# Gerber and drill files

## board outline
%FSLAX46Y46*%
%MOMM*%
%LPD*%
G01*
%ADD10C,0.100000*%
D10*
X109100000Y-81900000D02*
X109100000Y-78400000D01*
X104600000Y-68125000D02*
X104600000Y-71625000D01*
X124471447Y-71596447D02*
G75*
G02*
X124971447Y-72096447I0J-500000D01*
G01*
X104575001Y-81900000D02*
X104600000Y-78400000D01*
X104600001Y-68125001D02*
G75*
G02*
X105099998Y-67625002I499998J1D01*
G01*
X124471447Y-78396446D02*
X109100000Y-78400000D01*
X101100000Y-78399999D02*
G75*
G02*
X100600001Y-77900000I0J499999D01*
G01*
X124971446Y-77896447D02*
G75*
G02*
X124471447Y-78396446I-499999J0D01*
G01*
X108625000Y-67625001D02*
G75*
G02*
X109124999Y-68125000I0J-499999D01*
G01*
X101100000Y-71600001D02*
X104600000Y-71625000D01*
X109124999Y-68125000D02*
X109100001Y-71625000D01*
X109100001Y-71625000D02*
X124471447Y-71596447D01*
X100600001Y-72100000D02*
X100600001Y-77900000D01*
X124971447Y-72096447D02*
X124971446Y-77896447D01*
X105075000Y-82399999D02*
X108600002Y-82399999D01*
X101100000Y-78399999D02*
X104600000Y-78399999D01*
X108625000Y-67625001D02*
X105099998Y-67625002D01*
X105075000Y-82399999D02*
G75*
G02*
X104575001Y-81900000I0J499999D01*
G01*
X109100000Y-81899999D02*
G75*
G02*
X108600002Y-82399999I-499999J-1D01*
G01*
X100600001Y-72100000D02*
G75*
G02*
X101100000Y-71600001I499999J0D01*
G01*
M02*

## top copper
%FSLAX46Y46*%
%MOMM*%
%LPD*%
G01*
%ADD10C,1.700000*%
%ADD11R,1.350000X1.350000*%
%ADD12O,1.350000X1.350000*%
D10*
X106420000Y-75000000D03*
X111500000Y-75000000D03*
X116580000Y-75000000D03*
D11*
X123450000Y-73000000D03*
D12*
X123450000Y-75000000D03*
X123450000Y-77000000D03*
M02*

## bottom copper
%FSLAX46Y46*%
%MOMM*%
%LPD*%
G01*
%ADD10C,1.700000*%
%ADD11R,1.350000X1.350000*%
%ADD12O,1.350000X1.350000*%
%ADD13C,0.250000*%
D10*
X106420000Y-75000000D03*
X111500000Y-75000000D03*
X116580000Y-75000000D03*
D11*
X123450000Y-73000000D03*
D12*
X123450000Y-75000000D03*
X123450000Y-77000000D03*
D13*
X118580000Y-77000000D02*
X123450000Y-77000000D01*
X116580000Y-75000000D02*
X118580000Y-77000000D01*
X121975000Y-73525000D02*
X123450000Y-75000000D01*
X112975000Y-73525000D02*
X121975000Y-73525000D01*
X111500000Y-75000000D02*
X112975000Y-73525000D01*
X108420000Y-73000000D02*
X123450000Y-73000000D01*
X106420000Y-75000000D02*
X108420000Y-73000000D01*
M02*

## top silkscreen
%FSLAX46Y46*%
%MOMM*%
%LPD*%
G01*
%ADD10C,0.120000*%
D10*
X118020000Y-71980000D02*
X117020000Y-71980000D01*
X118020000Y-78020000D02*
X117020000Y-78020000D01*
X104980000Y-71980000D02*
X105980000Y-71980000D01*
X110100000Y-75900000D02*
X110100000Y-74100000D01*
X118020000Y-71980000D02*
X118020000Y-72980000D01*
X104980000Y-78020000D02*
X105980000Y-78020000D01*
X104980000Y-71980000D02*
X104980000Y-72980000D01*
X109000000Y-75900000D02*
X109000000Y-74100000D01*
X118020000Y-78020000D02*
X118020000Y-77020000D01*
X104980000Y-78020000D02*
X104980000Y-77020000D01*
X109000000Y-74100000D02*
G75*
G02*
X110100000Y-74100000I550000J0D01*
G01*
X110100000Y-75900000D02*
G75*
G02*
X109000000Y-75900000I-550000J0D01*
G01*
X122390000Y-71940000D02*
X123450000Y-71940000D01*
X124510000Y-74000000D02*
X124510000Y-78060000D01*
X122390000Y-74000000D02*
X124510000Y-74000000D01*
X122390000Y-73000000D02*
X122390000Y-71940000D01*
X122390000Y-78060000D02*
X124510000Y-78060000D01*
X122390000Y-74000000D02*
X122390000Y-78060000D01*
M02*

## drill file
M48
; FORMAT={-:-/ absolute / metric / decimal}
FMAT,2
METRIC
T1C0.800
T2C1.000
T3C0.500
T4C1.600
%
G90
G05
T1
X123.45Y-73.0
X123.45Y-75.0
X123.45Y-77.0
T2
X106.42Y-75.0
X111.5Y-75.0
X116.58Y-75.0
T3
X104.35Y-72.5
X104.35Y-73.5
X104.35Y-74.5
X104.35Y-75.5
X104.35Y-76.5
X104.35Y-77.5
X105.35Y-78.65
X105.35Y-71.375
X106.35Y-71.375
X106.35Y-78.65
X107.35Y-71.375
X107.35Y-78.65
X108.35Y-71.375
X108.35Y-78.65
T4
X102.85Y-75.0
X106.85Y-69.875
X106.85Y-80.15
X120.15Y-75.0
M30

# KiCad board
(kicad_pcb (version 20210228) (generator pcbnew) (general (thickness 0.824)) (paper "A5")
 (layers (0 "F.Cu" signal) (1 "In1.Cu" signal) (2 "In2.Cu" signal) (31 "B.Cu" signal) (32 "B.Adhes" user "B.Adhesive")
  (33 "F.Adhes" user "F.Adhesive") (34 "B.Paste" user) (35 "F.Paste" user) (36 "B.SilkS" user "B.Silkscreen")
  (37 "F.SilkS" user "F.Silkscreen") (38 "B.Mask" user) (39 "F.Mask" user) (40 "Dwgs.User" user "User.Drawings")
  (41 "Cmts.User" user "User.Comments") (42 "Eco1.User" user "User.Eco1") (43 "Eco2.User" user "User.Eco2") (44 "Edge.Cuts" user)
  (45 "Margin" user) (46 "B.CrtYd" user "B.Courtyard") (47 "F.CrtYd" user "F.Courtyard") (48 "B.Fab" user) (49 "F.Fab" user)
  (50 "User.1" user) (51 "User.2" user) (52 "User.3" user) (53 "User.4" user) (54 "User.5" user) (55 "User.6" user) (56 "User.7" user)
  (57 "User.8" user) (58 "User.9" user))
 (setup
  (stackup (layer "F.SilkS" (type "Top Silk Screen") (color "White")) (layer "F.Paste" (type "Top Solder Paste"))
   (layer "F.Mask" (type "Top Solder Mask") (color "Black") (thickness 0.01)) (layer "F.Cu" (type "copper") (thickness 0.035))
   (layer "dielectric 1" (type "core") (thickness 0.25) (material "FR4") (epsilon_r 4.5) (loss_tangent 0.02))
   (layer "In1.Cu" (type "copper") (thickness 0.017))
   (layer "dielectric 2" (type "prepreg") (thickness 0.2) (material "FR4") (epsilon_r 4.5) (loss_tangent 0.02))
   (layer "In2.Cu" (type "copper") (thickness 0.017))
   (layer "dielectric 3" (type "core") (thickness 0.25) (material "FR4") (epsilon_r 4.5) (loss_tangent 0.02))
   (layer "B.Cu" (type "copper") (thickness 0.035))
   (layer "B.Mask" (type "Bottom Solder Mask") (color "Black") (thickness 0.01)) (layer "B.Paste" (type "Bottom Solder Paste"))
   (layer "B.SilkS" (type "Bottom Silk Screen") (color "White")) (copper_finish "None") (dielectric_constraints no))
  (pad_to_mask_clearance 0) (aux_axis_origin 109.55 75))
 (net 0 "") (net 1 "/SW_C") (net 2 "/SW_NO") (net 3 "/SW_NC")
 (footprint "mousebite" (layer "F.Cu") (at 104.35 73.5)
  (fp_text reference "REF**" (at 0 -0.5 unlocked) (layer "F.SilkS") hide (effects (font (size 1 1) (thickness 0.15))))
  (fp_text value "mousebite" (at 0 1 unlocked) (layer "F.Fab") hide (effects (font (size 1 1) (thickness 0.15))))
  (pad "" np_thru_hole circle (at 0 0) (size 0.5 0.5) (drill 0.5) (layers F&B.Cu *.Mask)))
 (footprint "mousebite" (layer "F.Cu") (at 105.350001 71.375 -90)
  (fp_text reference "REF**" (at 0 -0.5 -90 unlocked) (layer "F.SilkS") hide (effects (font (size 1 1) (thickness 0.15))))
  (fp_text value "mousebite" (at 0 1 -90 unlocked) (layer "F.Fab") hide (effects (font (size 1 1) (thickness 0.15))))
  (pad "" np_thru_hole circle (at 0 0 270) (size 0.5 0.5) (drill 0.5) (layers F&B.Cu *.Mask)))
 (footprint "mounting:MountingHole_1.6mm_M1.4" (layer "F.Cu") (at 106.85 69.875001 -90)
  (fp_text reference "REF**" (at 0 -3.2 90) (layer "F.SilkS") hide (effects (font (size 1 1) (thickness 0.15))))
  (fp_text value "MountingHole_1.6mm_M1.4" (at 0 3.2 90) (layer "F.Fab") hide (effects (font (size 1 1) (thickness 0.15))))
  (pad "" np_thru_hole circle (at 0 0 270) (locked) (size 1.6 1.6) (drill 1.6) (layers F&B.Cu *.Mask)))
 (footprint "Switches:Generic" (layer "F.Cu") (at 111.5 75)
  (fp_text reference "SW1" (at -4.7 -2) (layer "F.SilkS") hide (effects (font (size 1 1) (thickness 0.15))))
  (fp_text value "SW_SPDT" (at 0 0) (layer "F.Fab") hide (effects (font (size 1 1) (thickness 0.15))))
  (fp_line (start 6.52 -3.02) (end 5.52 -3.02) (layer "F.SilkS") (width 0.12))
  (fp_line (start 6.52 3.02) (end 5.52 3.02) (layer "F.SilkS") (width 0.12))
  (fp_line (start -6.52 -3.02) (end -5.52 -3.02) (layer "F.SilkS") (width 0.12))
  (fp_line (start -1.4 0.9) (end -1.4 -0.9) (layer "F.SilkS") (width 0.12))
  (fp_line (start 6.52 -3.02) (end 6.52 -2.02) (layer "F.SilkS") (width 0.12))
  (fp_line (start -6.52 3.02) (end -5.52 3.02) (layer "F.SilkS") (width 0.12))
  (fp_line (start -6.52 -3.02) (end -6.52 -2.02) (layer "F.SilkS") (width 0.12))
  (fp_line (start -2.5 0.9) (end -2.5 -0.9) (layer "F.SilkS") (width 0.12))
  (fp_line (start 6.52 3.02) (end 6.52 2.02) (layer "F.SilkS") (width 0.12))
  (fp_line (start -6.52 3.02) (end -6.52 2.02) (layer "F.SilkS") (width 0.12))
  (fp_arc (start -1.95 -0.9) (end -1.4 -0.9) (angle -180) (layer "F.SilkS") (width 0.12))
  (fp_arc (start -1.95 0.9) (end -2.5 0.9) (angle -180) (layer "F.SilkS") (width 0.12))
  (pad "1" thru_hole circle (at -5.08 0) (locked) (size 1.7 1.7) (drill 1) (layers *.Cu *.Mask) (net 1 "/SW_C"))
  (pad "2" thru_hole circle (at 0 0) (locked) (size 1.7 1.7) (drill 1) (layers *.Cu *.Mask) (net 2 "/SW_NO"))
  (pad "3" thru_hole circle (at 5.08 0) (locked) (size 1.7 1.7) (drill 1) (layers *.Cu *.Mask) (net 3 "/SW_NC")))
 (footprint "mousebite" (layer "F.Cu") (at 104.35 75.5)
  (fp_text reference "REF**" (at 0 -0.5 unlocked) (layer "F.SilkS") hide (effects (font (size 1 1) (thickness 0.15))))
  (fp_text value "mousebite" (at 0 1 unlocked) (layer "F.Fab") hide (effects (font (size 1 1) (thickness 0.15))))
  (pad "" np_thru_hole circle (at 0 0) (size 0.5 0.5) (drill 0.5) (layers F&B.Cu *.Mask)))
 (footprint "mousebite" (layer "F.Cu") (at 104.35 74.5)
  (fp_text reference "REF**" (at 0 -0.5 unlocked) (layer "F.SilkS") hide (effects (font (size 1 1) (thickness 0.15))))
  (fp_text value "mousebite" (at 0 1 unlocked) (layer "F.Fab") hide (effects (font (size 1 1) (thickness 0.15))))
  (pad "" np_thru_hole circle (at 0 0) (size 0.5 0.5) (drill 0.5) (layers F&B.Cu *.Mask)))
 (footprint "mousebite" (layer "F.Cu") (at 104.35 76.5)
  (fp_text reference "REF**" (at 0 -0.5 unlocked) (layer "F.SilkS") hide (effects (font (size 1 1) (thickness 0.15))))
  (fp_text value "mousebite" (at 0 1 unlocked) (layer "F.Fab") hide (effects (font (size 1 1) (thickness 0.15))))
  (pad "" np_thru_hole circle (at 0 0) (size 0.5 0.5) (drill 0.5) (layers F&B.Cu *.Mask)))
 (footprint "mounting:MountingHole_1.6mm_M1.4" (layer "F.Cu") (at 120.15 75)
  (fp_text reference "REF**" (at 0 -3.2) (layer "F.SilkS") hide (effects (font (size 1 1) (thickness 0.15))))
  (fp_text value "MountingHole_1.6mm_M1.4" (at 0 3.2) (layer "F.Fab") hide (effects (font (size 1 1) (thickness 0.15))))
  (pad "" np_thru_hole circle (at 0 0) (locked) (size 1.6 1.6) (drill 1.6) (layers F&B.Cu *.Mask)))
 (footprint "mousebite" (layer "F.Cu") (at 104.35 72.5)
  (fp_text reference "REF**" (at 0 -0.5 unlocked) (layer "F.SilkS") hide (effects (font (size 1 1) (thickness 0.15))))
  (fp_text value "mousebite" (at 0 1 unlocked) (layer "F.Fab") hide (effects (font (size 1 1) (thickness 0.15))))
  (pad "" np_thru_hole circle (at 0 0) (size 0.5 0.5) (drill 0.5) (layers F&B.Cu *.Mask)))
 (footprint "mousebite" (layer "F.Cu") (at 107.35 78.65 90)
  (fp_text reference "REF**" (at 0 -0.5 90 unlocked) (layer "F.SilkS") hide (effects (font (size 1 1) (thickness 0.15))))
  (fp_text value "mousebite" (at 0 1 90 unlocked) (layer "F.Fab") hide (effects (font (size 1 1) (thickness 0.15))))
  (pad "" np_thru_hole circle (at 0 0 90) (size 0.5 0.5) (drill 0.5) (layers F&B.Cu *.Mask)))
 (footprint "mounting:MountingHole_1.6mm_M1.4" (layer "F.Cu") (at 102.85 75)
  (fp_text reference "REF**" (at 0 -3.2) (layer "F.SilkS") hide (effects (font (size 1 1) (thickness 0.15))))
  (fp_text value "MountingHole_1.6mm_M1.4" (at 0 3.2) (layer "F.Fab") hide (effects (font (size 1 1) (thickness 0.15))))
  (pad "" np_thru_hole circle (at 0 0) (locked) (size 1.6 1.6) (drill 1.6) (layers F&B.Cu *.Mask)))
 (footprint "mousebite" (layer "F.Cu") (at 108.349999 78.65 90)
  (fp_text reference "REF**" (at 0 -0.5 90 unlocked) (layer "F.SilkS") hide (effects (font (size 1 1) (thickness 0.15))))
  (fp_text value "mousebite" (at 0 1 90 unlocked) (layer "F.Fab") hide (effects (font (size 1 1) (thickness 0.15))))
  (pad "" np_thru_hole circle (at 0 0 90) (size 0.5 0.5) (drill 0.5) (layers F&B.Cu *.Mask)))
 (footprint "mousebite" (layer "F.Cu") (at 107.35 71.375 -90)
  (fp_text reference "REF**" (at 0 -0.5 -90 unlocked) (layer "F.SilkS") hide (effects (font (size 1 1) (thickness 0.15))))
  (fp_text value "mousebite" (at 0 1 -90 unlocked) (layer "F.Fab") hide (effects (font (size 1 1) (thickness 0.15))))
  (pad "" np_thru_hole circle (at 0 0 270) (size 0.5 0.5) (drill 0.5) (layers F&B.Cu *.Mask)))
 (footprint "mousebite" (layer "F.Cu") (at 106.35 78.65 90)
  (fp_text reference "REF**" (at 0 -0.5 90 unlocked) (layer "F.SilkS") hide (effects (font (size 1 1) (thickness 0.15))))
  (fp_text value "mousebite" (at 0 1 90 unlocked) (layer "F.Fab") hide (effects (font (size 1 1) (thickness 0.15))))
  (pad "" np_thru_hole circle (at 0 0 90) (size 0.5 0.5) (drill 0.5) (layers F&B.Cu *.Mask)))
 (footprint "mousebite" (layer "F.Cu") (at 105.35 78.65 90)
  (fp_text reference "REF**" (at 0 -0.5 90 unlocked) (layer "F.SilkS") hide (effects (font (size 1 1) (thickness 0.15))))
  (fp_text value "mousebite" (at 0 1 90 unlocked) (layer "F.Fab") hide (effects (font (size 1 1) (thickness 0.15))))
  (pad "" np_thru_hole circle (at 0 0 90) (size 0.5 0.5) (drill 0.5) (layers F&B.Cu *.Mask)))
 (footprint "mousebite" (layer "F.Cu") (at 106.35 71.375 -90)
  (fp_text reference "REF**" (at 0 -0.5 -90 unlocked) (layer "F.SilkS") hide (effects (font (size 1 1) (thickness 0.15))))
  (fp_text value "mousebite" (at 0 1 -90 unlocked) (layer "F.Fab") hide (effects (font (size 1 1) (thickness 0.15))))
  (pad "" np_thru_hole circle (at 0 0 270) (size 0.5 0.5) (drill 0.5) (layers F&B.Cu *.Mask)))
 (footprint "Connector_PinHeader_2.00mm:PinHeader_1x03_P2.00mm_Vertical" (layer "F.Cu") (at 123.45 73)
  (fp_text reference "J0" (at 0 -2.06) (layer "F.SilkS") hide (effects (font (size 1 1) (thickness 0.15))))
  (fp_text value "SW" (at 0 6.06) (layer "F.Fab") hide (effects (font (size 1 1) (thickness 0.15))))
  (fp_line (start -1.06 -1.06) (end 0 -1.06) (layer "F.SilkS") (width 0.12))
  (fp_line (start 1.06 1) (end 1.06 5.06) (layer "F.SilkS") (width 0.12))
  (fp_line (start -1.06 1) (end 1.06 1) (layer "F.SilkS") (width 0.12))
  (fp_line (start -1.06 0) (end -1.06 -1.06) (layer "F.SilkS") (width 0.12))
  (fp_line (start -1.06 5.06) (end 1.06 5.06) (layer "F.SilkS") (width 0.12))
  (fp_line (start -1.06 1) (end -1.06 5.06) (layer "F.SilkS") (width 0.12))
  (pad "1" thru_hole rect (at 0 0) (locked) (size 1.35 1.35) (drill 0.8) (layers *.Cu *.Mask) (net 1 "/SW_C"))
  (pad "2" thru_hole oval (at 0 2) (locked) (size 1.35 1.35) (drill 0.8) (layers *.Cu *.Mask) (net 2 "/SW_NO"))
  (pad "3" thru_hole oval (at 0 4) (locked) (size 1.35 1.35) (drill 0.8) (layers *.Cu *.Mask) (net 3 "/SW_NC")))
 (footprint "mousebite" (layer "F.Cu") (at 108.349999 71.375 -90)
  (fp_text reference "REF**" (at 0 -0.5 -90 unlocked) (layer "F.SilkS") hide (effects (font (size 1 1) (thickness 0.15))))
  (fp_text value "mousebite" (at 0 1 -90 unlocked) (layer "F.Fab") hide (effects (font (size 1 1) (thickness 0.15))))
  (pad "" np_thru_hole circle (at 0 0 270) (size 0.5 0.5) (drill 0.5) (layers F&B.Cu *.Mask)))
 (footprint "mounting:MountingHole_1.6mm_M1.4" (layer "F.Cu") (at 106.85 80.149999 90)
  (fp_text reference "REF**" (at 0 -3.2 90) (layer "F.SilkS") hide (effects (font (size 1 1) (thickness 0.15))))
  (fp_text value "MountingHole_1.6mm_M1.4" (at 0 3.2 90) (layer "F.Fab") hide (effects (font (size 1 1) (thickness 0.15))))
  (pad "" np_thru_hole circle (at 0 0 90) (locked) (size 1.6 1.6) (drill 1.6) (layers F&B.Cu *.Mask)))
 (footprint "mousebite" (layer "F.Cu") (at 104.35 77.5)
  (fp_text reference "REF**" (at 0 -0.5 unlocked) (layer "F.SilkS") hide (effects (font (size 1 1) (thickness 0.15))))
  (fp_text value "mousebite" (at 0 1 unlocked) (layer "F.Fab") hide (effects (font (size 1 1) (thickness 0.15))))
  (pad "" np_thru_hole circle (at 0 0) (size 0.5 0.5) (drill 0.5) (layers F&B.Cu *.Mask)))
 (gr_line (start 109.1 81.9) (end 109.1 78.4) (layer "Edge.Cuts") (width 0.1))
 (gr_line (start 104.6 68.125) (end 104.6 71.625) (layer "Edge.Cuts") (width 0.1))
 (gr_arc (start 124.471447 72.096447) (end 124.971447 72.096447) (angle -90) (layer "Edge.Cuts") (width 0.1))
 (gr_line (start 104.575001 81.9) (end 104.6 78.4) (layer "Edge.Cuts") (width 0.1))
 (gr_arc (start 105.099999 68.125) (end 105.099998 67.625002) (angle -90) (layer "Edge.Cuts") (width 0.1))
 (gr_line (start 124.471447 78.396446) (end 109.1 78.4) (layer "Edge.Cuts") (width 0.1))
 (gr_arc (start 101.1 77.9) (end 100.600001 77.9) (angle -90) (layer "Edge.Cuts") (width 0.1))
 (gr_arc (start 124.471447 77.896447) (end 124.471447 78.396446) (angle -90) (layer "Edge.Cuts") (width 0.1))
 (gr_arc (start 108.625 68.125) (end 109.124999 68.125) (angle -90) (layer "Edge.Cuts") (width 0.1))
 (gr_line (start 101.1 71.600001) (end 104.6 71.625) (layer "Edge.Cuts") (width 0.1))
 (gr_line (start 109.124999 68.125) (end 109.100001 71.625) (layer "Edge.Cuts") (width 0.1))
 (gr_line (start 109.100001 71.625) (end 124.471447 71.596447) (layer "Edge.Cuts") (width 0.1))
 (gr_line (start 100.600001 72.1) (end 100.600001 77.9) (layer "Edge.Cuts") (width 0.1))
 (gr_line (start 124.971447 72.096447) (end 124.971446 77.896447) (layer "Edge.Cuts") (width 0.1))
 (gr_line (start 105.075 82.399999) (end 108.600002 82.399999) (layer "Edge.Cuts") (width 0.1))
 (gr_line (start 101.1 78.399999) (end 104.6 78.399999) (layer "Edge.Cuts") (width 0.1))
 (gr_line (start 108.625 67.625001) (end 105.099998 67.625002) (layer "Edge.Cuts") (width 0.1))
 (gr_arc (start 105.075 81.9) (end 104.575001 81.9) (angle -90) (layer "Edge.Cuts") (width 0.1))
 (gr_arc (start 108.600001 81.9) (end 108.600002 82.399999) (angle -90) (layer "Edge.Cuts") (width 0.1))
 (gr_arc (start 101.1 72.1) (end 101.1 71.600001) (angle -90) (layer "Edge.Cuts") (width 0.1))
 (segment (start 118.58 77) (end 123.45 77) (width 0.25) (layer "B.Cu") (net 3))
 (segment (start 116.58 75) (end 118.58 77) (width 0.25) (layer "B.Cu") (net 3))
 (segment (start 121.975 73.525) (end 123.45 75) (width 0.25) (layer "B.Cu") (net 2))
 (segment (start 112.975 73.525) (end 121.975 73.525) (width 0.25) (layer "B.Cu") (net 2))
 (segment (start 111.5 75) (end 112.975 73.525) (width 0.25) (layer "B.Cu") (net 2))
 (segment (start 108.42 73) (end 123.45 73) (width 0.25) (layer "B.Cu") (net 1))
 (segment (start 106.42 75) (end 108.42 73) (width 0.25) (layer "B.Cu") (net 1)))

